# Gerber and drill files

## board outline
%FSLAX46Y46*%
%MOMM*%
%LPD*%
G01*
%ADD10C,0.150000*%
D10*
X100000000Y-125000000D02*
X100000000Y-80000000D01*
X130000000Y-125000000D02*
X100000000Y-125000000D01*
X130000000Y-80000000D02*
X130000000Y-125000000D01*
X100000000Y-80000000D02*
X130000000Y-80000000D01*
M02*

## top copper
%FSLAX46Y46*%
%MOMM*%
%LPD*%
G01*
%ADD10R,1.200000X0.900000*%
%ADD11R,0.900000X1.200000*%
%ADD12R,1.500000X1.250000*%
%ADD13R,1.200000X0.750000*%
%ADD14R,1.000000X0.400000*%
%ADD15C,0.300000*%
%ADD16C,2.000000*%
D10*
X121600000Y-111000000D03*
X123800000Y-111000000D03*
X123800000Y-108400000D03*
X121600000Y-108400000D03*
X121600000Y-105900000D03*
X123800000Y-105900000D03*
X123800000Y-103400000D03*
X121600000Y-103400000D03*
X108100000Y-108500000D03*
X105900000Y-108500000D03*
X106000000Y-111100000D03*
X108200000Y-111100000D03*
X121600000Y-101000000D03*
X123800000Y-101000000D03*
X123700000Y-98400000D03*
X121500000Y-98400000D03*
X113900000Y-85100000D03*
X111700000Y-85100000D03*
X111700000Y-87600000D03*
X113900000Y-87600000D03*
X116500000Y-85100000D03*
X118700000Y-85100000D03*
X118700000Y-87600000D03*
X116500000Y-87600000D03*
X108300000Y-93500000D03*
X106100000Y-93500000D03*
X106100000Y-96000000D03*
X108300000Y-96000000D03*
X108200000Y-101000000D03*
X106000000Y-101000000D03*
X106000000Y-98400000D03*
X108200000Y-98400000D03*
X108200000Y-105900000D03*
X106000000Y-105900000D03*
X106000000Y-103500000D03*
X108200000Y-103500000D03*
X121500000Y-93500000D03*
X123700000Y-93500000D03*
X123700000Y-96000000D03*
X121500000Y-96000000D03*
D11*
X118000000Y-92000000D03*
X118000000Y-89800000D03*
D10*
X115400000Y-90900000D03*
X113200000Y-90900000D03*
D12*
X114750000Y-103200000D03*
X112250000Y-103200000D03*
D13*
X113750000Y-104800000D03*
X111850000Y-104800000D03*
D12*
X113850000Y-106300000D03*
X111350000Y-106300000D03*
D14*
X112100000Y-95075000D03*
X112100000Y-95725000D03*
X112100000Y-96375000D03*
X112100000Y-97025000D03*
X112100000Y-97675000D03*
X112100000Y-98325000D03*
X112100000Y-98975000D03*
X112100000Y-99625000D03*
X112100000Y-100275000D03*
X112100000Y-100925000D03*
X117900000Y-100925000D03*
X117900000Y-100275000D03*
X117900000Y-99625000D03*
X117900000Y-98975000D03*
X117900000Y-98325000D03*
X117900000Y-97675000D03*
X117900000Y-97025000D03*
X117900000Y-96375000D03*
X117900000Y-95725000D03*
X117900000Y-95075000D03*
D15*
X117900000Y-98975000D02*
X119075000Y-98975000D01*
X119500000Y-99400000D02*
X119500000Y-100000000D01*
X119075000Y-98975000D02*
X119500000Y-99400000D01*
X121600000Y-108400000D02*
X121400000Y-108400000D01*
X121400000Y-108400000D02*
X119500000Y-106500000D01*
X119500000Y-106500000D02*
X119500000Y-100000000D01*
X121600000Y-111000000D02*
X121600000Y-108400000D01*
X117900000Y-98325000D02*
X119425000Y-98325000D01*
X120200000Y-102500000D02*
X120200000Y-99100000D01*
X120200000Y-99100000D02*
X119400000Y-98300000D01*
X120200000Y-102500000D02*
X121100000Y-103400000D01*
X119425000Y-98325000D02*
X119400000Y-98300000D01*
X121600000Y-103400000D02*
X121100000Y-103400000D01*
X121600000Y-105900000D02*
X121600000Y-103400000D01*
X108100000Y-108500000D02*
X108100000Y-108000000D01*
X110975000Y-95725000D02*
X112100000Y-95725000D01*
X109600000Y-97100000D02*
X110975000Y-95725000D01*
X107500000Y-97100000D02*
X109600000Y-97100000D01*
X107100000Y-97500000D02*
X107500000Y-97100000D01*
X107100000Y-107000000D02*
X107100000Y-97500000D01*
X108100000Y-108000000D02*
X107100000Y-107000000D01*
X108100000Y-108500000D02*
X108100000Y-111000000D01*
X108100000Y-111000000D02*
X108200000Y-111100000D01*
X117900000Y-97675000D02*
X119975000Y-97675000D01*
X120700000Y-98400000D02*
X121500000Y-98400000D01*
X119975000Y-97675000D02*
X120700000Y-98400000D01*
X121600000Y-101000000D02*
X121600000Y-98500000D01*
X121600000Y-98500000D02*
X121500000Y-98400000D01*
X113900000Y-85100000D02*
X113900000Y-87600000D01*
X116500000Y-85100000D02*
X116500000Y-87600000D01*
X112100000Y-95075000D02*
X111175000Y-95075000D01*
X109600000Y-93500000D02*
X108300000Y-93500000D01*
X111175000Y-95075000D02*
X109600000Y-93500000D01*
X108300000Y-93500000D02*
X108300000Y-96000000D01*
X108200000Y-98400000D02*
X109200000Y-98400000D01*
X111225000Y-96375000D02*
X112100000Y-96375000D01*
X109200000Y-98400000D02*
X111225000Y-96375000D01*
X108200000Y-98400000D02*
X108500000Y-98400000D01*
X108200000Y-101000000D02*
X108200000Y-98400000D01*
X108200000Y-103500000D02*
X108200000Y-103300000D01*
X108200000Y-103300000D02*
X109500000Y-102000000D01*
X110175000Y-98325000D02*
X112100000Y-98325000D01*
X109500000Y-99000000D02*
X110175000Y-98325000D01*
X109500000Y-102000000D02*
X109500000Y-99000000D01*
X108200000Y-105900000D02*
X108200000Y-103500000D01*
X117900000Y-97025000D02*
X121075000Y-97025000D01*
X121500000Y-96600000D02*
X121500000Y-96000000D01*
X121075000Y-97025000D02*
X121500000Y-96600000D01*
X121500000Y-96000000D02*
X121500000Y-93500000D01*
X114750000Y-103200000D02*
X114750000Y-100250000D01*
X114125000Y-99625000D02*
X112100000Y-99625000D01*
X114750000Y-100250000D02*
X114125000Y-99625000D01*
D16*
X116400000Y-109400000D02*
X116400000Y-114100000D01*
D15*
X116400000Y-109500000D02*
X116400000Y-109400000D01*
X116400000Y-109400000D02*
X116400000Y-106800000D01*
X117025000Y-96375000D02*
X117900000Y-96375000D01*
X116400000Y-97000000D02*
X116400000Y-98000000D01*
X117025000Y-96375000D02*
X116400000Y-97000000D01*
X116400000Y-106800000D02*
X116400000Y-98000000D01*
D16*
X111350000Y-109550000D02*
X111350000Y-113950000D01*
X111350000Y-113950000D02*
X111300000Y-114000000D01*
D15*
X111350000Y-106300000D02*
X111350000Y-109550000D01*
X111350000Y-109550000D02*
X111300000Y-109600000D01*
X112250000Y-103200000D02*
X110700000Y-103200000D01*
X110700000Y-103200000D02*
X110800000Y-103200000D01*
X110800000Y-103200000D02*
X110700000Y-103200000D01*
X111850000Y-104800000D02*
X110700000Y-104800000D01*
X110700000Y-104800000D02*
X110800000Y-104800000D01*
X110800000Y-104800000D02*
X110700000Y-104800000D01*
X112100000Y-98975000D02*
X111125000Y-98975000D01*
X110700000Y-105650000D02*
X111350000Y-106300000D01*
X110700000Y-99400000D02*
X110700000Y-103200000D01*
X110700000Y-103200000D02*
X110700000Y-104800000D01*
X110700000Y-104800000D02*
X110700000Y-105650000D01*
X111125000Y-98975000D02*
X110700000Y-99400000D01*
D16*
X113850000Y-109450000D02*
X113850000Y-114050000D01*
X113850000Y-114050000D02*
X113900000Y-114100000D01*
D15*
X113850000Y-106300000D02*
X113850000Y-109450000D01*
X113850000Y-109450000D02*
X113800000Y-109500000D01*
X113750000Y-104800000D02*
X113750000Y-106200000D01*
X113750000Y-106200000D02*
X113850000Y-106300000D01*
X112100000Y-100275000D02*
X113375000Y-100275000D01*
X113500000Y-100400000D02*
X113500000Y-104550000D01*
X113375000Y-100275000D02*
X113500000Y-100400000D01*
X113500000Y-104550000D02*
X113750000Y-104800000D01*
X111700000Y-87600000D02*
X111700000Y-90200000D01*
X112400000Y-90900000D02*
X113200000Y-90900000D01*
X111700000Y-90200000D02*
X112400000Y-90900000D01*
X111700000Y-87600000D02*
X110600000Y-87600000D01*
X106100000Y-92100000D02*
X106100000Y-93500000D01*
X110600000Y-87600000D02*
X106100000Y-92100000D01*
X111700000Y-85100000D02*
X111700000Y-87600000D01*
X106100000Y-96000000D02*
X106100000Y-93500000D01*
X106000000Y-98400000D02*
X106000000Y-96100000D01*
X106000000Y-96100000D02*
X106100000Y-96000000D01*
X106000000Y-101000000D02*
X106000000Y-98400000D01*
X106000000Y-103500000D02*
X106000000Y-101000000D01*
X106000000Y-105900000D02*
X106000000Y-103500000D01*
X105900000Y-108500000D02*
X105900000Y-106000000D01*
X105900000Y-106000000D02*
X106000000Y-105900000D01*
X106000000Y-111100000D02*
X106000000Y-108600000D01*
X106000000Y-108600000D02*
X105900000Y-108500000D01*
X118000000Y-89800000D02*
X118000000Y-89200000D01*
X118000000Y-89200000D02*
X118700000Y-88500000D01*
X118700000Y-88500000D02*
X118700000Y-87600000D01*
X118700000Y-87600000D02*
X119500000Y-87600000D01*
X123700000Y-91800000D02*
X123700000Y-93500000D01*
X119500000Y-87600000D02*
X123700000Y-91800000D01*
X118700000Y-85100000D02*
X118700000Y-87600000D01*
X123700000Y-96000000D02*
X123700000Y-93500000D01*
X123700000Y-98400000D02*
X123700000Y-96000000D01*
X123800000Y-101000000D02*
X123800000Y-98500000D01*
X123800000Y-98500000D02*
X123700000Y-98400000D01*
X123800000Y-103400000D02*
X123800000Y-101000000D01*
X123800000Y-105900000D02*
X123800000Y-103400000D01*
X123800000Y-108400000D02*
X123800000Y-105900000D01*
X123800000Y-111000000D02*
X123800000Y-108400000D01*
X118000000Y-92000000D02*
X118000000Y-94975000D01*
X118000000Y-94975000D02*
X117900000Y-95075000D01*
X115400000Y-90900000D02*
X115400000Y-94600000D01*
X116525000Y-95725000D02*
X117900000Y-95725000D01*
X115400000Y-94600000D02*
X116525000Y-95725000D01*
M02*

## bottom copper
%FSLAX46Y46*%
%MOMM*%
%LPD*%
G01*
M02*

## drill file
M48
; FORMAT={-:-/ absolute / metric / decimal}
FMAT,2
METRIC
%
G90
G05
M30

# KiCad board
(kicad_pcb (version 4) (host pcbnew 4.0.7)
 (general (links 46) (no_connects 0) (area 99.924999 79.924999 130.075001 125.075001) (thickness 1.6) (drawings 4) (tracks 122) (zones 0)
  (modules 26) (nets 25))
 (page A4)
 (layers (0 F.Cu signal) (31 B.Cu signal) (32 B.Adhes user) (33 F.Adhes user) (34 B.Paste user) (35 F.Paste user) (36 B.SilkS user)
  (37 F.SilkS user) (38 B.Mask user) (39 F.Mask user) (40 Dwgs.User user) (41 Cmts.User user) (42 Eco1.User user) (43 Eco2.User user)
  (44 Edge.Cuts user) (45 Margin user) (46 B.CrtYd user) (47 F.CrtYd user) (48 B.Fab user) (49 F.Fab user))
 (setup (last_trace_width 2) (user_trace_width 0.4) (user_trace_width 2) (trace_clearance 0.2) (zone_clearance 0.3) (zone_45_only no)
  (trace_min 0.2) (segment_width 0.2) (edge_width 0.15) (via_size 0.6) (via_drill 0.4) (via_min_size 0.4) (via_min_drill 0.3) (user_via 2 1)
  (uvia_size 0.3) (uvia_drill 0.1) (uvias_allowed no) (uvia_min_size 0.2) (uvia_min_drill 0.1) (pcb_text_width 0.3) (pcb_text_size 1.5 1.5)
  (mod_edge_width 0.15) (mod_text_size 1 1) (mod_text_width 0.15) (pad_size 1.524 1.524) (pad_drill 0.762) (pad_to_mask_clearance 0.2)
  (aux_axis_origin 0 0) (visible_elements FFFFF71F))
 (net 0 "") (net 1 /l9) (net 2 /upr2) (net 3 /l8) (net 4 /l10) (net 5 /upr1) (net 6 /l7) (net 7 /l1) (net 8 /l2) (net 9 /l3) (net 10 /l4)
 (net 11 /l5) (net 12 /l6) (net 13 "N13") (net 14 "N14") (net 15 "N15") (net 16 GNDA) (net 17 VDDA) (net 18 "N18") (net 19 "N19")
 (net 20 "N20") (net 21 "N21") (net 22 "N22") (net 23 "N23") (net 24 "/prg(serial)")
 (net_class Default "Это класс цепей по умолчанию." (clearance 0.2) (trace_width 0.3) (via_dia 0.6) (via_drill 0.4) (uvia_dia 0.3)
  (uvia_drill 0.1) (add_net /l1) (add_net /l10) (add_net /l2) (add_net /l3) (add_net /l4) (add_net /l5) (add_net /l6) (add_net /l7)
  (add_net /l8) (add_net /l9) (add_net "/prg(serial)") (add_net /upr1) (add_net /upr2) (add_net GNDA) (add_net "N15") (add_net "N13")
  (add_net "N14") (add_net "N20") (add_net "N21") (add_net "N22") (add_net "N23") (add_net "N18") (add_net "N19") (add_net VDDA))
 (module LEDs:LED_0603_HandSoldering (layer F.Cu) (at 122.7 111)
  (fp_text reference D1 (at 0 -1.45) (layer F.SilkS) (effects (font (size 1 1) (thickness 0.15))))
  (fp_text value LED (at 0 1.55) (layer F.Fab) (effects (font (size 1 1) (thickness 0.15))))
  (pad 1 smd rect (at -1.1 0) (size 1.2 0.9) (layers F.Cu F.Paste F.Mask) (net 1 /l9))
  (pad 2 smd rect (at 1.1 0) (size 1.2 0.9) (layers F.Cu F.Paste F.Mask) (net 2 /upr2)))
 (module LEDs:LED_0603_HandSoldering (layer F.Cu) (at 122.7 108.4 180)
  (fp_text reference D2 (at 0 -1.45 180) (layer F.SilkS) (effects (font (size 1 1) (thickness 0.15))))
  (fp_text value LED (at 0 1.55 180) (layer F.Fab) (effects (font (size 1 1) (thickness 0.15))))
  (pad 1 smd rect (at -1.1 0 180) (size 1.2 0.9) (layers F.Cu F.Paste F.Mask) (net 2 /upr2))
  (pad 2 smd rect (at 1.1 0 180) (size 1.2 0.9) (layers F.Cu F.Paste F.Mask) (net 1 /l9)))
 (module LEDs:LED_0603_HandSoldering (layer F.Cu) (at 122.7 105.9)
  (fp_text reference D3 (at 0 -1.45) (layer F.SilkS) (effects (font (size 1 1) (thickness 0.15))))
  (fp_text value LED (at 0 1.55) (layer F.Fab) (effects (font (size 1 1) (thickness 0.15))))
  (pad 1 smd rect (at -1.1 0) (size 1.2 0.9) (layers F.Cu F.Paste F.Mask) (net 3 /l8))
  (pad 2 smd rect (at 1.1 0) (size 1.2 0.9) (layers F.Cu F.Paste F.Mask) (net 2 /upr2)))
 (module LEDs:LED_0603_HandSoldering (layer F.Cu) (at 122.7 103.4 180)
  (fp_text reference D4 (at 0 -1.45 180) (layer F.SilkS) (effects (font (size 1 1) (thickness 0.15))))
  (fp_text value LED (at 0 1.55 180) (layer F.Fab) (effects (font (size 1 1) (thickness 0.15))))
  (pad 1 smd rect (at -1.1 0 180) (size 1.2 0.9) (layers F.Cu F.Paste F.Mask) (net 2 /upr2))
  (pad 2 smd rect (at 1.1 0 180) (size 1.2 0.9) (layers F.Cu F.Paste F.Mask) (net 3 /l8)))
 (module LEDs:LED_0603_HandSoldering (layer F.Cu) (at 107 108.5 180)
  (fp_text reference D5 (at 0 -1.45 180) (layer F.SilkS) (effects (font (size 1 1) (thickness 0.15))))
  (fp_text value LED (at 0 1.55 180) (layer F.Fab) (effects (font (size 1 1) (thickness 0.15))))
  (pad 1 smd rect (at -1.1 0 180) (size 1.2 0.9) (layers F.Cu F.Paste F.Mask) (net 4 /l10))
  (pad 2 smd rect (at 1.1 0 180) (size 1.2 0.9) (layers F.Cu F.Paste F.Mask) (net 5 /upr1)))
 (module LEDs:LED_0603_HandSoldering (layer F.Cu) (at 107.1 111.1)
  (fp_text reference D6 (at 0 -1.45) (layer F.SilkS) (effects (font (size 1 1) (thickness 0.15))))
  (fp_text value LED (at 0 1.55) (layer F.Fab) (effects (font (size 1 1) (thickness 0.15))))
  (pad 1 smd rect (at -1.1 0) (size 1.2 0.9) (layers F.Cu F.Paste F.Mask) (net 5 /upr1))
  (pad 2 smd rect (at 1.1 0) (size 1.2 0.9) (layers F.Cu F.Paste F.Mask) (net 4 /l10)))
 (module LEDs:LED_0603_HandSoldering (layer F.Cu) (at 122.7 101)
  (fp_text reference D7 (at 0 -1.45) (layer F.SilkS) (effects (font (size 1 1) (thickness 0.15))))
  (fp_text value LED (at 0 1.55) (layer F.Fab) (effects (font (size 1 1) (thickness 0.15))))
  (pad 1 smd rect (at -1.1 0) (size 1.2 0.9) (layers F.Cu F.Paste F.Mask) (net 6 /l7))
  (pad 2 smd rect (at 1.1 0) (size 1.2 0.9) (layers F.Cu F.Paste F.Mask) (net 2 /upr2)))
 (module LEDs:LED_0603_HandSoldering (layer F.Cu) (at 122.6 98.4 180)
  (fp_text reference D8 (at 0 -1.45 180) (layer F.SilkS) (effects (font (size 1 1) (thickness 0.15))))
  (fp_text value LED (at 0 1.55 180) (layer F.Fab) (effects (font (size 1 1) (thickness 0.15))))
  (pad 1 smd rect (at -1.1 0 180) (size 1.2 0.9) (layers F.Cu F.Paste F.Mask) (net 2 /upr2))
  (pad 2 smd rect (at 1.1 0 180) (size 1.2 0.9) (layers F.Cu F.Paste F.Mask) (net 6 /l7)))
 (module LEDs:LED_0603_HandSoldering (layer F.Cu) (at 112.8 85.1 180)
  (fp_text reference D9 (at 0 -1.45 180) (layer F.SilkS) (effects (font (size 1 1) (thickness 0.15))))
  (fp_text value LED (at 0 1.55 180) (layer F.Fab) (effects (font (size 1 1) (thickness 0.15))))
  (pad 1 smd rect (at -1.1 0 180) (size 1.2 0.9) (layers F.Cu F.Paste F.Mask) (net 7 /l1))
  (pad 2 smd rect (at 1.1 0 180) (size 1.2 0.9) (layers F.Cu F.Paste F.Mask) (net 5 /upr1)))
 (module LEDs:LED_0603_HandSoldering (layer F.Cu) (at 112.8 87.6)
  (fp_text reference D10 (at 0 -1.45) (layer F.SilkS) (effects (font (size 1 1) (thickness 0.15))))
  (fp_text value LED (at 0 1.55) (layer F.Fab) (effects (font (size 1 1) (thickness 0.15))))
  (pad 1 smd rect (at -1.1 0) (size 1.2 0.9) (layers F.Cu F.Paste F.Mask) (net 5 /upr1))
  (pad 2 smd rect (at 1.1 0) (size 1.2 0.9) (layers F.Cu F.Paste F.Mask) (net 7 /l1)))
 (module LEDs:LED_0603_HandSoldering (layer F.Cu) (at 117.6 85.1)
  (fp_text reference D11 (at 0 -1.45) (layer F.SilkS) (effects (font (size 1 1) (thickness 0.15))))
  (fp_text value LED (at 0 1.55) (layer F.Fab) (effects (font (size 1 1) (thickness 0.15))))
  (pad 1 smd rect (at -1.1 0) (size 1.2 0.9) (layers F.Cu F.Paste F.Mask) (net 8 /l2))
  (pad 2 smd rect (at 1.1 0) (size 1.2 0.9) (layers F.Cu F.Paste F.Mask) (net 2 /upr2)))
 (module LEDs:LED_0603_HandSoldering (layer F.Cu) (at 117.6 87.6 180)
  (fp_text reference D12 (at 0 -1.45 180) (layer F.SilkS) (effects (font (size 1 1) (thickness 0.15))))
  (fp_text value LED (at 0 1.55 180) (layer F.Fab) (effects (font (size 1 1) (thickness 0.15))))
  (pad 1 smd rect (at -1.1 0 180) (size 1.2 0.9) (layers F.Cu F.Paste F.Mask) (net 2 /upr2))
  (pad 2 smd rect (at 1.1 0 180) (size 1.2 0.9) (layers F.Cu F.Paste F.Mask) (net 8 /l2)))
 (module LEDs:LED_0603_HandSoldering (layer F.Cu) (at 107.2 93.5 180)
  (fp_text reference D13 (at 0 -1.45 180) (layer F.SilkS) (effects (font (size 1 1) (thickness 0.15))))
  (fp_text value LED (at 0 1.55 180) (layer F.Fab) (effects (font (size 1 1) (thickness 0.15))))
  (pad 1 smd rect (at -1.1 0 180) (size 1.2 0.9) (layers F.Cu F.Paste F.Mask) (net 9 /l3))
  (pad 2 smd rect (at 1.1 0 180) (size 1.2 0.9) (layers F.Cu F.Paste F.Mask) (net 5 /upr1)))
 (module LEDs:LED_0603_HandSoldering (layer F.Cu) (at 107.2 96)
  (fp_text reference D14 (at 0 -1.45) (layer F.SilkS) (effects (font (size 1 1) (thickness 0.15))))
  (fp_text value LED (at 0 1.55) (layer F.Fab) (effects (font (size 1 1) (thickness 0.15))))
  (pad 1 smd rect (at -1.1 0) (size 1.2 0.9) (layers F.Cu F.Paste F.Mask) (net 5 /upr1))
  (pad 2 smd rect (at 1.1 0) (size 1.2 0.9) (layers F.Cu F.Paste F.Mask) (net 9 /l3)))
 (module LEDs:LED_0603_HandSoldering (layer F.Cu) (at 107.1 101 180)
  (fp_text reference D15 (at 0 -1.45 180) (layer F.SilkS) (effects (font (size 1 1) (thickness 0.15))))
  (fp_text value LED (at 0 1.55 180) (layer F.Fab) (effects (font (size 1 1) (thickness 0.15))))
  (pad 1 smd rect (at -1.1 0 180) (size 1.2 0.9) (layers F.Cu F.Paste F.Mask) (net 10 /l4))
  (pad 2 smd rect (at 1.1 0 180) (size 1.2 0.9) (layers F.Cu F.Paste F.Mask) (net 5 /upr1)))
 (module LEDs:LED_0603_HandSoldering (layer F.Cu) (at 107.1 98.4)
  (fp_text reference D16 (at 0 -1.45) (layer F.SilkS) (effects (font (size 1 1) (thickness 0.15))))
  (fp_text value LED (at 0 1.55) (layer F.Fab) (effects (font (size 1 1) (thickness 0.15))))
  (pad 1 smd rect (at -1.1 0) (size 1.2 0.9) (layers F.Cu F.Paste F.Mask) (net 5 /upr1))
  (pad 2 smd rect (at 1.1 0) (size 1.2 0.9) (layers F.Cu F.Paste F.Mask) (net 10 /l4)))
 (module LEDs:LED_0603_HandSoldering (layer F.Cu) (at 107.1 105.9 180)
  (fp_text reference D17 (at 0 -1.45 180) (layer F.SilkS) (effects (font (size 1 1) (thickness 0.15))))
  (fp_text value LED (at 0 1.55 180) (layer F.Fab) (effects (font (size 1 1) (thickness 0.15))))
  (pad 1 smd rect (at -1.1 0 180) (size 1.2 0.9) (layers F.Cu F.Paste F.Mask) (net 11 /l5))
  (pad 2 smd rect (at 1.1 0 180) (size 1.2 0.9) (layers F.Cu F.Paste F.Mask) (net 5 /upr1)))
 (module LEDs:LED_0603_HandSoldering (layer F.Cu) (at 107.1 103.5)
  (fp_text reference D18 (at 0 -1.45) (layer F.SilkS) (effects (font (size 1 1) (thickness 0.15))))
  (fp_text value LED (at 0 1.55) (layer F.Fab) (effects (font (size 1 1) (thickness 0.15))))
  (pad 1 smd rect (at -1.1 0) (size 1.2 0.9) (layers F.Cu F.Paste F.Mask) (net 5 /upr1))
  (pad 2 smd rect (at 1.1 0) (size 1.2 0.9) (layers F.Cu F.Paste F.Mask) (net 11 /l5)))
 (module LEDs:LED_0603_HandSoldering (layer F.Cu) (at 122.6 93.5)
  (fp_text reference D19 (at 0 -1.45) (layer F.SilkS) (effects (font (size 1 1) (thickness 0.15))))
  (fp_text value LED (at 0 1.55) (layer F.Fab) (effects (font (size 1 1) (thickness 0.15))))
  (pad 1 smd rect (at -1.1 0) (size 1.2 0.9) (layers F.Cu F.Paste F.Mask) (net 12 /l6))
  (pad 2 smd rect (at 1.1 0) (size 1.2 0.9) (layers F.Cu F.Paste F.Mask) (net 2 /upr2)))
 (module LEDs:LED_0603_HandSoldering (layer F.Cu) (at 122.6 96 180)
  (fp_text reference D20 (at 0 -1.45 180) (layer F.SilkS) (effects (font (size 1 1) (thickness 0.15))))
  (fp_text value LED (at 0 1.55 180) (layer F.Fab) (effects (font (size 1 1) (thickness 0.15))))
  (pad 1 smd rect (at -1.1 0 180) (size 1.2 0.9) (layers F.Cu F.Paste F.Mask) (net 2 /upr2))
  (pad 2 smd rect (at 1.1 0 180) (size 1.2 0.9) (layers F.Cu F.Paste F.Mask) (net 12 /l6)))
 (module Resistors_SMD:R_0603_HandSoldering (layer F.Cu) (at 118 90.9 90)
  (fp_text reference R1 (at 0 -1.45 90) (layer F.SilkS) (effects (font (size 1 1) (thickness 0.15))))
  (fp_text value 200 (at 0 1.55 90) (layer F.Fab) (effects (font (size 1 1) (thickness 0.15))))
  (pad 1 smd rect (at -1.1 0 90) (size 1.2 0.9) (layers F.Cu F.Paste F.Mask) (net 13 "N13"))
  (pad 2 smd rect (at 1.1 0 90) (size 1.2 0.9) (layers F.Cu F.Paste F.Mask) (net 2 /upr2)))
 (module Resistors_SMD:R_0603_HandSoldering (layer F.Cu) (at 114.3 90.9 180)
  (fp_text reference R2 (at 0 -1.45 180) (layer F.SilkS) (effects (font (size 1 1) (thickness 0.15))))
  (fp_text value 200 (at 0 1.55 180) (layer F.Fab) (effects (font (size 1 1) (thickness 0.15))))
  (pad 1 smd rect (at -1.1 0 180) (size 1.2 0.9) (layers F.Cu F.Paste F.Mask) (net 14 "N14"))
  (pad 2 smd rect (at 1.1 0 180) (size 1.2 0.9) (layers F.Cu F.Paste F.Mask) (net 5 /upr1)))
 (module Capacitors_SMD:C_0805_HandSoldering (layer F.Cu) (at 113.5 103.2 180)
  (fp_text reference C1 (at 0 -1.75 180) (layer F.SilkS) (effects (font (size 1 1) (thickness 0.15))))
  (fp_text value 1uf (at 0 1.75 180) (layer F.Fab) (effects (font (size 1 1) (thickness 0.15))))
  (pad 1 smd rect (at -1.25 0 180) (size 1.5 1.25) (layers F.Cu F.Paste F.Mask) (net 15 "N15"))
  (pad 2 smd rect (at 1.25 0 180) (size 1.5 1.25) (layers F.Cu F.Paste F.Mask) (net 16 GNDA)))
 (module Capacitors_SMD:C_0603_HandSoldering (layer F.Cu) (at 112.8 104.8 180)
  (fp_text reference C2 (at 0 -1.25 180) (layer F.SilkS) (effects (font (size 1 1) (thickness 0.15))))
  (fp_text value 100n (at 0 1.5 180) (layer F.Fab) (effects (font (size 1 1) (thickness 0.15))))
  (pad 1 smd rect (at -0.95 0 180) (size 1.2 0.75) (layers F.Cu F.Paste F.Mask) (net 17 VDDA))
  (pad 2 smd rect (at 0.95 0 180) (size 1.2 0.75) (layers F.Cu F.Paste F.Mask) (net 16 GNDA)))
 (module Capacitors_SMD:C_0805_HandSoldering (layer F.Cu) (at 112.6 106.3 180)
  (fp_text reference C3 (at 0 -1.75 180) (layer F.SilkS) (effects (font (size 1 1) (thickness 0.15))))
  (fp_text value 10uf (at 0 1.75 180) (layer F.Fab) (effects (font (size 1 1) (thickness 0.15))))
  (pad 1 smd rect (at -1.25 0 180) (size 1.5 1.25) (layers F.Cu F.Paste F.Mask) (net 17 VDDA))
  (pad 2 smd rect (at 1.25 0 180) (size 1.5 1.25) (layers F.Cu F.Paste F.Mask) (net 16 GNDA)))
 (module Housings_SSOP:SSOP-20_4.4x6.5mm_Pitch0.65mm (layer F.Cu) (at 115 98)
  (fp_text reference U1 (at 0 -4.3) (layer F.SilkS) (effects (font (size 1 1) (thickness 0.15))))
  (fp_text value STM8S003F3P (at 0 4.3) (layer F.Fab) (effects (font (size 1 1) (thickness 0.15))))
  (pad 1 smd rect (at -2.9 -2.925) (size 1 0.4) (layers F.Cu F.Paste F.Mask) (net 9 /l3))
  (pad 2 smd rect (at -2.9 -2.275) (size 1 0.4) (layers F.Cu F.Paste F.Mask) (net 4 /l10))
  (pad 3 smd rect (at -2.9 -1.625) (size 1 0.4) (layers F.Cu F.Paste F.Mask) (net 10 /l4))
  (pad 4 smd rect (at -2.9 -0.975) (size 1 0.4) (layers F.Cu F.Paste F.Mask) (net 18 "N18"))
  (pad 5 smd rect (at -2.9 -0.325) (size 1 0.4) (layers F.Cu F.Paste F.Mask) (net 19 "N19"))
  (pad 6 smd rect (at -2.9 0.325) (size 1 0.4) (layers F.Cu F.Paste F.Mask) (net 11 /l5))
  (pad 7 smd rect (at -2.9 0.975) (size 1 0.4) (layers F.Cu F.Paste F.Mask) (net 16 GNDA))
  (pad 8 smd rect (at -2.9 1.625) (size 1 0.4) (layers F.Cu F.Paste F.Mask) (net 15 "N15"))
  (pad 9 smd rect (at -2.9 2.275) (size 1 0.4) (layers F.Cu F.Paste F.Mask) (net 17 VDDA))
  (pad 10 smd rect (at -2.9 2.925) (size 1 0.4) (layers F.Cu F.Paste F.Mask) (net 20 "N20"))
  (pad 11 smd rect (at 2.9 2.925) (size 1 0.4) (layers F.Cu F.Paste F.Mask) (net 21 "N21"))
  (pad 12 smd rect (at 2.9 2.275) (size 1 0.4) (layers F.Cu F.Paste F.Mask) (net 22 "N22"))
  (pad 13 smd rect (at 2.9 1.625) (size 1 0.4) (layers F.Cu F.Paste F.Mask) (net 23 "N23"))
  (pad 14 smd rect (at 2.9 0.975) (size 1 0.4) (layers F.Cu F.Paste F.Mask) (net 1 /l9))
  (pad 15 smd rect (at 2.9 0.325) (size 1 0.4) (layers F.Cu F.Paste F.Mask) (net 3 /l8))
  (pad 16 smd rect (at 2.9 -0.325) (size 1 0.4) (layers F.Cu F.Paste F.Mask) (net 6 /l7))
  (pad 17 smd rect (at 2.9 -0.975) (size 1 0.4) (layers F.Cu F.Paste F.Mask) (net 12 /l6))
  (pad 18 smd rect (at 2.9 -1.625) (size 1 0.4) (layers F.Cu F.Paste F.Mask) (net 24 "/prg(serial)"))
  (pad 19 smd rect (at 2.9 -2.275) (size 1 0.4) (layers F.Cu F.Paste F.Mask) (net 14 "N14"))
  (pad 20 smd rect (at 2.9 -2.925) (size 1 0.4) (layers F.Cu F.Paste F.Mask) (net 13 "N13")))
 (gr_line (start 100 125) (end 100 80) (angle 90) (layer Edge.Cuts) (width 0.15))
 (gr_line (start 130 125) (end 100 125) (angle 90) (layer Edge.Cuts) (width 0.15))
 (gr_line (start 130 80) (end 130 125) (angle 90) (layer Edge.Cuts) (width 0.15))
 (gr_line (start 100 80) (end 130 80) (angle 90) (layer Edge.Cuts) (width 0.15))
 (segment (start 117.9 98.975) (end 119.075 98.975) (width 0.3) (layer F.Cu) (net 1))
 (segment (start 119.5 99.4) (end 119.5 100) (width 0.3) (layer F.Cu) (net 1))
 (segment (start 119.075 98.975) (end 119.5 99.4) (width 0.3) (layer F.Cu) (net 1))
 (segment (start 121.6 108.4) (end 121.4 108.4) (width 0.3) (layer F.Cu) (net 1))
 (segment (start 121.4 108.4) (end 119.5 106.5) (width 0.3) (layer F.Cu) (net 1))
 (segment (start 119.5 106.5) (end 119.5 100) (width 0.3) (layer F.Cu) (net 1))
 (segment (start 121.6 111) (end 121.6 108.4) (width 0.3) (layer F.Cu) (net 1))
 (segment (start 117.9 98.325) (end 119.425 98.325) (width 0.3) (layer F.Cu) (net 3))
 (segment (start 120.2 102.5) (end 120.2 99.1) (width 0.3) (layer F.Cu) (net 3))
 (segment (start 120.2 99.1) (end 119.4 98.3) (width 0.3) (layer F.Cu) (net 3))
 (segment (start 120.2 102.5) (end 121.1 103.4) (width 0.3) (layer F.Cu) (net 3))
 (segment (start 119.425 98.325) (end 119.4 98.3) (width 0.3) (layer F.Cu) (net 3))
 (segment (start 121.6 103.4) (end 121.1 103.4) (width 0.3) (layer F.Cu) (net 3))
 (segment (start 121.6 105.9) (end 121.6 103.4) (width 0.3) (layer F.Cu) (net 3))
 (segment (start 108.1 108.5) (end 108.1 108) (width 0.3) (layer F.Cu) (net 4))
 (segment (start 110.975 95.725) (end 112.1 95.725) (width 0.3) (layer F.Cu) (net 4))
 (segment (start 109.6 97.1) (end 110.975 95.725) (width 0.3) (layer F.Cu) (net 4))
 (segment (start 107.5 97.1) (end 109.6 97.1) (width 0.3) (layer F.Cu) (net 4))
 (segment (start 107.1 97.5) (end 107.5 97.1) (width 0.3) (layer F.Cu) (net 4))
 (segment (start 107.1 107) (end 107.1 97.5) (width 0.3) (layer F.Cu) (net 4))
 (segment (start 108.1 108) (end 107.1 107) (width 0.3) (layer F.Cu) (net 4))
 (segment (start 108.1 108.5) (end 108.1 111) (width 0.3) (layer F.Cu) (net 4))
 (segment (start 108.1 111) (end 108.2 111.1) (width 0.3) (layer F.Cu) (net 4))
 (segment (start 117.9 97.675) (end 119.975 97.675) (width 0.3) (layer F.Cu) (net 6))
 (segment (start 120.7 98.4) (end 121.5 98.4) (width 0.3) (layer F.Cu) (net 6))
 (segment (start 119.975 97.675) (end 120.7 98.4) (width 0.3) (layer F.Cu) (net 6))
 (segment (start 121.6 101) (end 121.6 98.5) (width 0.3) (layer F.Cu) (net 6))
 (segment (start 121.6 98.5) (end 121.5 98.4) (width 0.3) (layer F.Cu) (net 6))
 (segment (start 113.9 85.1) (end 113.9 87.6) (width 0.3) (layer F.Cu) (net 7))
 (segment (start 116.5 85.1) (end 116.5 87.6) (width 0.3) (layer F.Cu) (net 8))
 (segment (start 112.1 95.075) (end 111.175 95.075) (width 0.3) (layer F.Cu) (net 9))
 (segment (start 109.6 93.5) (end 108.3 93.5) (width 0.3) (layer F.Cu) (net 9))
 (segment (start 111.175 95.075) (end 109.6 93.5) (width 0.3) (layer F.Cu) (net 9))
 (segment (start 108.3 93.5) (end 108.3 96) (width 0.3) (layer F.Cu) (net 9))
 (segment (start 108.2 98.4) (end 109.2 98.4) (width 0.3) (layer F.Cu) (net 10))
 (segment (start 111.225 96.375) (end 112.1 96.375) (width 0.3) (layer F.Cu) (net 10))
 (segment (start 109.2 98.4) (end 111.225 96.375) (width 0.3) (layer F.Cu) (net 10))
 (segment (start 108.2 98.4) (end 108.5 98.4) (width 0.3) (layer F.Cu) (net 10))
 (segment (start 108.2 101) (end 108.2 98.4) (width 0.3) (layer F.Cu) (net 10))
 (segment (start 108.2 103.5) (end 108.2 103.3) (width 0.3) (layer F.Cu) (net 11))
 (segment (start 108.2 103.3) (end 109.5 102) (width 0.3) (layer F.Cu) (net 11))
 (segment (start 110.175 98.325) (end 112.1 98.325) (width 0.3) (layer F.Cu) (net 11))
 (segment (start 109.5 99) (end 110.175 98.325) (width 0.3) (layer F.Cu) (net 11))
 (segment (start 109.5 102) (end 109.5 99) (width 0.3) (layer F.Cu) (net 11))
 (segment (start 108.2 105.9) (end 108.2 103.5) (width 0.3) (layer F.Cu) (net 11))
 (segment (start 117.9 97.025) (end 121.075 97.025) (width 0.3) (layer F.Cu) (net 12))
 (segment (start 121.5 96.6) (end 121.5 96) (width 0.3) (layer F.Cu) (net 12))
 (segment (start 121.075 97.025) (end 121.5 96.6) (width 0.3) (layer F.Cu) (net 12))
 (segment (start 121.5 96) (end 121.5 93.5) (width 0.3) (layer F.Cu) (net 12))
 (segment (start 114.75 103.2) (end 114.75 100.25) (width 0.3) (layer F.Cu) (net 15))
 (segment (start 114.125 99.625) (end 112.1 99.625) (width 0.3) (layer F.Cu) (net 15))
 (segment (start 114.75 100.25) (end 114.125 99.625) (width 0.3) (layer F.Cu) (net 15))
 (segment (start 116.4 109.4) (end 116.4 114.1) (width 2) (layer F.Cu) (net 24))
 (segment (start 116.4 109.5) (end 116.4 109.4) (width 0.3) (layer F.Cu) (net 24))
 (segment (start 116.4 109.4) (end 116.4 106.8) (width 0.3) (layer F.Cu) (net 24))
 (segment (start 117.025 96.375) (end 117.9 96.375) (width 0.3) (layer F.Cu) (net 24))
 (segment (start 116.4 97) (end 116.4 98) (width 0.3) (layer F.Cu) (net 24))
 (segment (start 117.025 96.375) (end 116.4 97) (width 0.3) (layer F.Cu) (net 24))
 (segment (start 116.4 106.8) (end 116.4 98) (width 0.3) (layer F.Cu) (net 24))
 (segment (start 111.35 109.55) (end 111.35 113.95) (width 2) (layer F.Cu) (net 16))
 (segment (start 111.35 113.95) (end 111.3 114) (width 2) (layer F.Cu) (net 16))
 (segment (start 111.35 106.3) (end 111.35 109.55) (width 0.3) (layer F.Cu) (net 16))
 (segment (start 111.35 109.55) (end 111.3 109.6) (width 0.3) (layer F.Cu) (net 16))
 (segment (start 112.25 103.2) (end 110.7 103.2) (width 0.3) (layer F.Cu) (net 16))
 (segment (start 110.7 103.2) (end 110.8 103.2) (width 0.3) (layer F.Cu) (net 16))
 (segment (start 110.8 103.2) (end 110.7 103.2) (width 0.3) (layer F.Cu) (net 16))
 (segment (start 111.85 104.8) (end 110.7 104.8) (width 0.3) (layer F.Cu) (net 16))
 (segment (start 110.7 104.8) (end 110.8 104.8) (width 0.3) (layer F.Cu) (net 16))
 (segment (start 110.8 104.8) (end 110.7 104.8) (width 0.3) (layer F.Cu) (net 16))
 (segment (start 112.1 98.975) (end 111.125 98.975) (width 0.3) (layer F.Cu) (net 16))
 (segment (start 110.7 105.65) (end 111.35 106.3) (width 0.3) (layer F.Cu) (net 16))
 (segment (start 110.7 99.4) (end 110.7 103.2) (width 0.3) (layer F.Cu) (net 16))
 (segment (start 110.7 103.2) (end 110.7 104.8) (width 0.3) (layer F.Cu) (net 16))
 (segment (start 110.7 104.8) (end 110.7 105.65) (width 0.3) (layer F.Cu) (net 16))
 (segment (start 111.125 98.975) (end 110.7 99.4) (width 0.3) (layer F.Cu) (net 16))
 (segment (start 113.85 109.45) (end 113.85 114.05) (width 2) (layer F.Cu) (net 17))
 (segment (start 113.85 114.05) (end 113.9 114.1) (width 2) (layer F.Cu) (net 17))
 (segment (start 113.85 106.3) (end 113.85 109.45) (width 0.3) (layer F.Cu) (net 17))
 (segment (start 113.85 109.45) (end 113.8 109.5) (width 0.3) (layer F.Cu) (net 17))
 (segment (start 113.75 104.8) (end 113.75 106.2) (width 0.3) (layer F.Cu) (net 17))
 (segment (start 113.75 106.2) (end 113.85 106.3) (width 0.3) (layer F.Cu) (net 17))
 (segment (start 112.1 100.275) (end 113.375 100.275) (width 0.3) (layer F.Cu) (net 17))
 (segment (start 113.5 100.4) (end 113.5 104.55) (width 0.3) (layer F.Cu) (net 17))
 (segment (start 113.375 100.275) (end 113.5 100.4) (width 0.3) (layer F.Cu) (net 17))
 (segment (start 113.5 104.55) (end 113.75 104.8) (width 0.3) (layer F.Cu) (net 17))
 (segment (start 111.7 87.6) (end 111.7 90.2) (width 0.3) (layer F.Cu) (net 5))
 (segment (start 112.4 90.9) (end 113.2 90.9) (width 0.3) (layer F.Cu) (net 5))
 (segment (start 111.7 90.2) (end 112.4 90.9) (width 0.3) (layer F.Cu) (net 5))
 (segment (start 111.7 87.6) (end 110.6 87.6) (width 0.3) (layer F.Cu) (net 5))
 (segment (start 106.1 92.1) (end 106.1 93.5) (width 0.3) (layer F.Cu) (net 5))
 (segment (start 110.6 87.6) (end 106.1 92.1) (width 0.3) (layer F.Cu) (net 5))
 (segment (start 111.7 85.1) (end 111.7 87.6) (width 0.3) (layer F.Cu) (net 5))
 (segment (start 106.1 96) (end 106.1 93.5) (width 0.3) (layer F.Cu) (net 5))
 (segment (start 106 98.4) (end 106 96.1) (width 0.3) (layer F.Cu) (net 5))
 (segment (start 106 96.1) (end 106.1 96) (width 0.3) (layer F.Cu) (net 5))
 (segment (start 106 101) (end 106 98.4) (width 0.3) (layer F.Cu) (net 5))
 (segment (start 106 103.5) (end 106 101) (width 0.3) (layer F.Cu) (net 5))
 (segment (start 106 105.9) (end 106 103.5) (width 0.3) (layer F.Cu) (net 5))
 (segment (start 105.9 108.5) (end 105.9 106) (width 0.3) (layer F.Cu) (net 5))
 (segment (start 105.9 106) (end 106 105.9) (width 0.3) (layer F.Cu) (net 5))
 (segment (start 106 111.1) (end 106 108.6) (width 0.3) (layer F.Cu) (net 5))
 (segment (start 106 108.6) (end 105.9 108.5) (width 0.3) (layer F.Cu) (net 5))
 (segment (start 118 89.8) (end 118 89.2) (width 0.3) (layer F.Cu) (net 2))
 (segment (start 118 89.2) (end 118.7 88.5) (width 0.3) (layer F.Cu) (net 2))
 (segment (start 118.7 88.5) (end 118.7 87.6) (width 0.3) (layer F.Cu) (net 2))
 (segment (start 118.7 87.6) (end 119.5 87.6) (width 0.3) (layer F.Cu) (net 2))
 (segment (start 123.7 91.8) (end 123.7 93.5) (width 0.3) (layer F.Cu) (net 2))
 (segment (start 119.5 87.6) (end 123.7 91.8) (width 0.3) (layer F.Cu) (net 2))
 (segment (start 118.7 85.1) (end 118.7 87.6) (width 0.3) (layer F.Cu) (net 2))
 (segment (start 123.7 96) (end 123.7 93.5) (width 0.3) (layer F.Cu) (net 2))
 (segment (start 123.7 98.4) (end 123.7 96) (width 0.3) (layer F.Cu) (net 2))
 (segment (start 123.8 101) (end 123.8 98.5) (width 0.3) (layer F.Cu) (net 2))
 (segment (start 123.8 98.5) (end 123.7 98.4) (width 0.3) (layer F.Cu) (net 2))
 (segment (start 123.8 103.4) (end 123.8 101) (width 0.3) (layer F.Cu) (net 2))
 (segment (start 123.8 105.9) (end 123.8 103.4) (width 0.3) (layer F.Cu) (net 2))
 (segment (start 123.8 108.4) (end 123.8 105.9) (width 0.3) (layer F.Cu) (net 2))
 (segment (start 123.8 111) (end 123.8 108.4) (width 0.3) (layer F.Cu) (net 2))
 (segment (start 118 92) (end 118 94.975) (width 0.3) (layer F.Cu) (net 13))
 (segment (start 118 94.975) (end 117.9 95.075) (width 0.3) (layer F.Cu) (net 13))
 (segment (start 115.4 90.9) (end 115.4 94.6) (width 0.3) (layer F.Cu) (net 14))
 (segment (start 116.525 95.725) (end 117.9 95.725) (width 0.3) (layer F.Cu) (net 14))
 (segment (start 115.4 94.6) (end 116.525 95.725) (width 0.3) (layer F.Cu) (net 14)))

